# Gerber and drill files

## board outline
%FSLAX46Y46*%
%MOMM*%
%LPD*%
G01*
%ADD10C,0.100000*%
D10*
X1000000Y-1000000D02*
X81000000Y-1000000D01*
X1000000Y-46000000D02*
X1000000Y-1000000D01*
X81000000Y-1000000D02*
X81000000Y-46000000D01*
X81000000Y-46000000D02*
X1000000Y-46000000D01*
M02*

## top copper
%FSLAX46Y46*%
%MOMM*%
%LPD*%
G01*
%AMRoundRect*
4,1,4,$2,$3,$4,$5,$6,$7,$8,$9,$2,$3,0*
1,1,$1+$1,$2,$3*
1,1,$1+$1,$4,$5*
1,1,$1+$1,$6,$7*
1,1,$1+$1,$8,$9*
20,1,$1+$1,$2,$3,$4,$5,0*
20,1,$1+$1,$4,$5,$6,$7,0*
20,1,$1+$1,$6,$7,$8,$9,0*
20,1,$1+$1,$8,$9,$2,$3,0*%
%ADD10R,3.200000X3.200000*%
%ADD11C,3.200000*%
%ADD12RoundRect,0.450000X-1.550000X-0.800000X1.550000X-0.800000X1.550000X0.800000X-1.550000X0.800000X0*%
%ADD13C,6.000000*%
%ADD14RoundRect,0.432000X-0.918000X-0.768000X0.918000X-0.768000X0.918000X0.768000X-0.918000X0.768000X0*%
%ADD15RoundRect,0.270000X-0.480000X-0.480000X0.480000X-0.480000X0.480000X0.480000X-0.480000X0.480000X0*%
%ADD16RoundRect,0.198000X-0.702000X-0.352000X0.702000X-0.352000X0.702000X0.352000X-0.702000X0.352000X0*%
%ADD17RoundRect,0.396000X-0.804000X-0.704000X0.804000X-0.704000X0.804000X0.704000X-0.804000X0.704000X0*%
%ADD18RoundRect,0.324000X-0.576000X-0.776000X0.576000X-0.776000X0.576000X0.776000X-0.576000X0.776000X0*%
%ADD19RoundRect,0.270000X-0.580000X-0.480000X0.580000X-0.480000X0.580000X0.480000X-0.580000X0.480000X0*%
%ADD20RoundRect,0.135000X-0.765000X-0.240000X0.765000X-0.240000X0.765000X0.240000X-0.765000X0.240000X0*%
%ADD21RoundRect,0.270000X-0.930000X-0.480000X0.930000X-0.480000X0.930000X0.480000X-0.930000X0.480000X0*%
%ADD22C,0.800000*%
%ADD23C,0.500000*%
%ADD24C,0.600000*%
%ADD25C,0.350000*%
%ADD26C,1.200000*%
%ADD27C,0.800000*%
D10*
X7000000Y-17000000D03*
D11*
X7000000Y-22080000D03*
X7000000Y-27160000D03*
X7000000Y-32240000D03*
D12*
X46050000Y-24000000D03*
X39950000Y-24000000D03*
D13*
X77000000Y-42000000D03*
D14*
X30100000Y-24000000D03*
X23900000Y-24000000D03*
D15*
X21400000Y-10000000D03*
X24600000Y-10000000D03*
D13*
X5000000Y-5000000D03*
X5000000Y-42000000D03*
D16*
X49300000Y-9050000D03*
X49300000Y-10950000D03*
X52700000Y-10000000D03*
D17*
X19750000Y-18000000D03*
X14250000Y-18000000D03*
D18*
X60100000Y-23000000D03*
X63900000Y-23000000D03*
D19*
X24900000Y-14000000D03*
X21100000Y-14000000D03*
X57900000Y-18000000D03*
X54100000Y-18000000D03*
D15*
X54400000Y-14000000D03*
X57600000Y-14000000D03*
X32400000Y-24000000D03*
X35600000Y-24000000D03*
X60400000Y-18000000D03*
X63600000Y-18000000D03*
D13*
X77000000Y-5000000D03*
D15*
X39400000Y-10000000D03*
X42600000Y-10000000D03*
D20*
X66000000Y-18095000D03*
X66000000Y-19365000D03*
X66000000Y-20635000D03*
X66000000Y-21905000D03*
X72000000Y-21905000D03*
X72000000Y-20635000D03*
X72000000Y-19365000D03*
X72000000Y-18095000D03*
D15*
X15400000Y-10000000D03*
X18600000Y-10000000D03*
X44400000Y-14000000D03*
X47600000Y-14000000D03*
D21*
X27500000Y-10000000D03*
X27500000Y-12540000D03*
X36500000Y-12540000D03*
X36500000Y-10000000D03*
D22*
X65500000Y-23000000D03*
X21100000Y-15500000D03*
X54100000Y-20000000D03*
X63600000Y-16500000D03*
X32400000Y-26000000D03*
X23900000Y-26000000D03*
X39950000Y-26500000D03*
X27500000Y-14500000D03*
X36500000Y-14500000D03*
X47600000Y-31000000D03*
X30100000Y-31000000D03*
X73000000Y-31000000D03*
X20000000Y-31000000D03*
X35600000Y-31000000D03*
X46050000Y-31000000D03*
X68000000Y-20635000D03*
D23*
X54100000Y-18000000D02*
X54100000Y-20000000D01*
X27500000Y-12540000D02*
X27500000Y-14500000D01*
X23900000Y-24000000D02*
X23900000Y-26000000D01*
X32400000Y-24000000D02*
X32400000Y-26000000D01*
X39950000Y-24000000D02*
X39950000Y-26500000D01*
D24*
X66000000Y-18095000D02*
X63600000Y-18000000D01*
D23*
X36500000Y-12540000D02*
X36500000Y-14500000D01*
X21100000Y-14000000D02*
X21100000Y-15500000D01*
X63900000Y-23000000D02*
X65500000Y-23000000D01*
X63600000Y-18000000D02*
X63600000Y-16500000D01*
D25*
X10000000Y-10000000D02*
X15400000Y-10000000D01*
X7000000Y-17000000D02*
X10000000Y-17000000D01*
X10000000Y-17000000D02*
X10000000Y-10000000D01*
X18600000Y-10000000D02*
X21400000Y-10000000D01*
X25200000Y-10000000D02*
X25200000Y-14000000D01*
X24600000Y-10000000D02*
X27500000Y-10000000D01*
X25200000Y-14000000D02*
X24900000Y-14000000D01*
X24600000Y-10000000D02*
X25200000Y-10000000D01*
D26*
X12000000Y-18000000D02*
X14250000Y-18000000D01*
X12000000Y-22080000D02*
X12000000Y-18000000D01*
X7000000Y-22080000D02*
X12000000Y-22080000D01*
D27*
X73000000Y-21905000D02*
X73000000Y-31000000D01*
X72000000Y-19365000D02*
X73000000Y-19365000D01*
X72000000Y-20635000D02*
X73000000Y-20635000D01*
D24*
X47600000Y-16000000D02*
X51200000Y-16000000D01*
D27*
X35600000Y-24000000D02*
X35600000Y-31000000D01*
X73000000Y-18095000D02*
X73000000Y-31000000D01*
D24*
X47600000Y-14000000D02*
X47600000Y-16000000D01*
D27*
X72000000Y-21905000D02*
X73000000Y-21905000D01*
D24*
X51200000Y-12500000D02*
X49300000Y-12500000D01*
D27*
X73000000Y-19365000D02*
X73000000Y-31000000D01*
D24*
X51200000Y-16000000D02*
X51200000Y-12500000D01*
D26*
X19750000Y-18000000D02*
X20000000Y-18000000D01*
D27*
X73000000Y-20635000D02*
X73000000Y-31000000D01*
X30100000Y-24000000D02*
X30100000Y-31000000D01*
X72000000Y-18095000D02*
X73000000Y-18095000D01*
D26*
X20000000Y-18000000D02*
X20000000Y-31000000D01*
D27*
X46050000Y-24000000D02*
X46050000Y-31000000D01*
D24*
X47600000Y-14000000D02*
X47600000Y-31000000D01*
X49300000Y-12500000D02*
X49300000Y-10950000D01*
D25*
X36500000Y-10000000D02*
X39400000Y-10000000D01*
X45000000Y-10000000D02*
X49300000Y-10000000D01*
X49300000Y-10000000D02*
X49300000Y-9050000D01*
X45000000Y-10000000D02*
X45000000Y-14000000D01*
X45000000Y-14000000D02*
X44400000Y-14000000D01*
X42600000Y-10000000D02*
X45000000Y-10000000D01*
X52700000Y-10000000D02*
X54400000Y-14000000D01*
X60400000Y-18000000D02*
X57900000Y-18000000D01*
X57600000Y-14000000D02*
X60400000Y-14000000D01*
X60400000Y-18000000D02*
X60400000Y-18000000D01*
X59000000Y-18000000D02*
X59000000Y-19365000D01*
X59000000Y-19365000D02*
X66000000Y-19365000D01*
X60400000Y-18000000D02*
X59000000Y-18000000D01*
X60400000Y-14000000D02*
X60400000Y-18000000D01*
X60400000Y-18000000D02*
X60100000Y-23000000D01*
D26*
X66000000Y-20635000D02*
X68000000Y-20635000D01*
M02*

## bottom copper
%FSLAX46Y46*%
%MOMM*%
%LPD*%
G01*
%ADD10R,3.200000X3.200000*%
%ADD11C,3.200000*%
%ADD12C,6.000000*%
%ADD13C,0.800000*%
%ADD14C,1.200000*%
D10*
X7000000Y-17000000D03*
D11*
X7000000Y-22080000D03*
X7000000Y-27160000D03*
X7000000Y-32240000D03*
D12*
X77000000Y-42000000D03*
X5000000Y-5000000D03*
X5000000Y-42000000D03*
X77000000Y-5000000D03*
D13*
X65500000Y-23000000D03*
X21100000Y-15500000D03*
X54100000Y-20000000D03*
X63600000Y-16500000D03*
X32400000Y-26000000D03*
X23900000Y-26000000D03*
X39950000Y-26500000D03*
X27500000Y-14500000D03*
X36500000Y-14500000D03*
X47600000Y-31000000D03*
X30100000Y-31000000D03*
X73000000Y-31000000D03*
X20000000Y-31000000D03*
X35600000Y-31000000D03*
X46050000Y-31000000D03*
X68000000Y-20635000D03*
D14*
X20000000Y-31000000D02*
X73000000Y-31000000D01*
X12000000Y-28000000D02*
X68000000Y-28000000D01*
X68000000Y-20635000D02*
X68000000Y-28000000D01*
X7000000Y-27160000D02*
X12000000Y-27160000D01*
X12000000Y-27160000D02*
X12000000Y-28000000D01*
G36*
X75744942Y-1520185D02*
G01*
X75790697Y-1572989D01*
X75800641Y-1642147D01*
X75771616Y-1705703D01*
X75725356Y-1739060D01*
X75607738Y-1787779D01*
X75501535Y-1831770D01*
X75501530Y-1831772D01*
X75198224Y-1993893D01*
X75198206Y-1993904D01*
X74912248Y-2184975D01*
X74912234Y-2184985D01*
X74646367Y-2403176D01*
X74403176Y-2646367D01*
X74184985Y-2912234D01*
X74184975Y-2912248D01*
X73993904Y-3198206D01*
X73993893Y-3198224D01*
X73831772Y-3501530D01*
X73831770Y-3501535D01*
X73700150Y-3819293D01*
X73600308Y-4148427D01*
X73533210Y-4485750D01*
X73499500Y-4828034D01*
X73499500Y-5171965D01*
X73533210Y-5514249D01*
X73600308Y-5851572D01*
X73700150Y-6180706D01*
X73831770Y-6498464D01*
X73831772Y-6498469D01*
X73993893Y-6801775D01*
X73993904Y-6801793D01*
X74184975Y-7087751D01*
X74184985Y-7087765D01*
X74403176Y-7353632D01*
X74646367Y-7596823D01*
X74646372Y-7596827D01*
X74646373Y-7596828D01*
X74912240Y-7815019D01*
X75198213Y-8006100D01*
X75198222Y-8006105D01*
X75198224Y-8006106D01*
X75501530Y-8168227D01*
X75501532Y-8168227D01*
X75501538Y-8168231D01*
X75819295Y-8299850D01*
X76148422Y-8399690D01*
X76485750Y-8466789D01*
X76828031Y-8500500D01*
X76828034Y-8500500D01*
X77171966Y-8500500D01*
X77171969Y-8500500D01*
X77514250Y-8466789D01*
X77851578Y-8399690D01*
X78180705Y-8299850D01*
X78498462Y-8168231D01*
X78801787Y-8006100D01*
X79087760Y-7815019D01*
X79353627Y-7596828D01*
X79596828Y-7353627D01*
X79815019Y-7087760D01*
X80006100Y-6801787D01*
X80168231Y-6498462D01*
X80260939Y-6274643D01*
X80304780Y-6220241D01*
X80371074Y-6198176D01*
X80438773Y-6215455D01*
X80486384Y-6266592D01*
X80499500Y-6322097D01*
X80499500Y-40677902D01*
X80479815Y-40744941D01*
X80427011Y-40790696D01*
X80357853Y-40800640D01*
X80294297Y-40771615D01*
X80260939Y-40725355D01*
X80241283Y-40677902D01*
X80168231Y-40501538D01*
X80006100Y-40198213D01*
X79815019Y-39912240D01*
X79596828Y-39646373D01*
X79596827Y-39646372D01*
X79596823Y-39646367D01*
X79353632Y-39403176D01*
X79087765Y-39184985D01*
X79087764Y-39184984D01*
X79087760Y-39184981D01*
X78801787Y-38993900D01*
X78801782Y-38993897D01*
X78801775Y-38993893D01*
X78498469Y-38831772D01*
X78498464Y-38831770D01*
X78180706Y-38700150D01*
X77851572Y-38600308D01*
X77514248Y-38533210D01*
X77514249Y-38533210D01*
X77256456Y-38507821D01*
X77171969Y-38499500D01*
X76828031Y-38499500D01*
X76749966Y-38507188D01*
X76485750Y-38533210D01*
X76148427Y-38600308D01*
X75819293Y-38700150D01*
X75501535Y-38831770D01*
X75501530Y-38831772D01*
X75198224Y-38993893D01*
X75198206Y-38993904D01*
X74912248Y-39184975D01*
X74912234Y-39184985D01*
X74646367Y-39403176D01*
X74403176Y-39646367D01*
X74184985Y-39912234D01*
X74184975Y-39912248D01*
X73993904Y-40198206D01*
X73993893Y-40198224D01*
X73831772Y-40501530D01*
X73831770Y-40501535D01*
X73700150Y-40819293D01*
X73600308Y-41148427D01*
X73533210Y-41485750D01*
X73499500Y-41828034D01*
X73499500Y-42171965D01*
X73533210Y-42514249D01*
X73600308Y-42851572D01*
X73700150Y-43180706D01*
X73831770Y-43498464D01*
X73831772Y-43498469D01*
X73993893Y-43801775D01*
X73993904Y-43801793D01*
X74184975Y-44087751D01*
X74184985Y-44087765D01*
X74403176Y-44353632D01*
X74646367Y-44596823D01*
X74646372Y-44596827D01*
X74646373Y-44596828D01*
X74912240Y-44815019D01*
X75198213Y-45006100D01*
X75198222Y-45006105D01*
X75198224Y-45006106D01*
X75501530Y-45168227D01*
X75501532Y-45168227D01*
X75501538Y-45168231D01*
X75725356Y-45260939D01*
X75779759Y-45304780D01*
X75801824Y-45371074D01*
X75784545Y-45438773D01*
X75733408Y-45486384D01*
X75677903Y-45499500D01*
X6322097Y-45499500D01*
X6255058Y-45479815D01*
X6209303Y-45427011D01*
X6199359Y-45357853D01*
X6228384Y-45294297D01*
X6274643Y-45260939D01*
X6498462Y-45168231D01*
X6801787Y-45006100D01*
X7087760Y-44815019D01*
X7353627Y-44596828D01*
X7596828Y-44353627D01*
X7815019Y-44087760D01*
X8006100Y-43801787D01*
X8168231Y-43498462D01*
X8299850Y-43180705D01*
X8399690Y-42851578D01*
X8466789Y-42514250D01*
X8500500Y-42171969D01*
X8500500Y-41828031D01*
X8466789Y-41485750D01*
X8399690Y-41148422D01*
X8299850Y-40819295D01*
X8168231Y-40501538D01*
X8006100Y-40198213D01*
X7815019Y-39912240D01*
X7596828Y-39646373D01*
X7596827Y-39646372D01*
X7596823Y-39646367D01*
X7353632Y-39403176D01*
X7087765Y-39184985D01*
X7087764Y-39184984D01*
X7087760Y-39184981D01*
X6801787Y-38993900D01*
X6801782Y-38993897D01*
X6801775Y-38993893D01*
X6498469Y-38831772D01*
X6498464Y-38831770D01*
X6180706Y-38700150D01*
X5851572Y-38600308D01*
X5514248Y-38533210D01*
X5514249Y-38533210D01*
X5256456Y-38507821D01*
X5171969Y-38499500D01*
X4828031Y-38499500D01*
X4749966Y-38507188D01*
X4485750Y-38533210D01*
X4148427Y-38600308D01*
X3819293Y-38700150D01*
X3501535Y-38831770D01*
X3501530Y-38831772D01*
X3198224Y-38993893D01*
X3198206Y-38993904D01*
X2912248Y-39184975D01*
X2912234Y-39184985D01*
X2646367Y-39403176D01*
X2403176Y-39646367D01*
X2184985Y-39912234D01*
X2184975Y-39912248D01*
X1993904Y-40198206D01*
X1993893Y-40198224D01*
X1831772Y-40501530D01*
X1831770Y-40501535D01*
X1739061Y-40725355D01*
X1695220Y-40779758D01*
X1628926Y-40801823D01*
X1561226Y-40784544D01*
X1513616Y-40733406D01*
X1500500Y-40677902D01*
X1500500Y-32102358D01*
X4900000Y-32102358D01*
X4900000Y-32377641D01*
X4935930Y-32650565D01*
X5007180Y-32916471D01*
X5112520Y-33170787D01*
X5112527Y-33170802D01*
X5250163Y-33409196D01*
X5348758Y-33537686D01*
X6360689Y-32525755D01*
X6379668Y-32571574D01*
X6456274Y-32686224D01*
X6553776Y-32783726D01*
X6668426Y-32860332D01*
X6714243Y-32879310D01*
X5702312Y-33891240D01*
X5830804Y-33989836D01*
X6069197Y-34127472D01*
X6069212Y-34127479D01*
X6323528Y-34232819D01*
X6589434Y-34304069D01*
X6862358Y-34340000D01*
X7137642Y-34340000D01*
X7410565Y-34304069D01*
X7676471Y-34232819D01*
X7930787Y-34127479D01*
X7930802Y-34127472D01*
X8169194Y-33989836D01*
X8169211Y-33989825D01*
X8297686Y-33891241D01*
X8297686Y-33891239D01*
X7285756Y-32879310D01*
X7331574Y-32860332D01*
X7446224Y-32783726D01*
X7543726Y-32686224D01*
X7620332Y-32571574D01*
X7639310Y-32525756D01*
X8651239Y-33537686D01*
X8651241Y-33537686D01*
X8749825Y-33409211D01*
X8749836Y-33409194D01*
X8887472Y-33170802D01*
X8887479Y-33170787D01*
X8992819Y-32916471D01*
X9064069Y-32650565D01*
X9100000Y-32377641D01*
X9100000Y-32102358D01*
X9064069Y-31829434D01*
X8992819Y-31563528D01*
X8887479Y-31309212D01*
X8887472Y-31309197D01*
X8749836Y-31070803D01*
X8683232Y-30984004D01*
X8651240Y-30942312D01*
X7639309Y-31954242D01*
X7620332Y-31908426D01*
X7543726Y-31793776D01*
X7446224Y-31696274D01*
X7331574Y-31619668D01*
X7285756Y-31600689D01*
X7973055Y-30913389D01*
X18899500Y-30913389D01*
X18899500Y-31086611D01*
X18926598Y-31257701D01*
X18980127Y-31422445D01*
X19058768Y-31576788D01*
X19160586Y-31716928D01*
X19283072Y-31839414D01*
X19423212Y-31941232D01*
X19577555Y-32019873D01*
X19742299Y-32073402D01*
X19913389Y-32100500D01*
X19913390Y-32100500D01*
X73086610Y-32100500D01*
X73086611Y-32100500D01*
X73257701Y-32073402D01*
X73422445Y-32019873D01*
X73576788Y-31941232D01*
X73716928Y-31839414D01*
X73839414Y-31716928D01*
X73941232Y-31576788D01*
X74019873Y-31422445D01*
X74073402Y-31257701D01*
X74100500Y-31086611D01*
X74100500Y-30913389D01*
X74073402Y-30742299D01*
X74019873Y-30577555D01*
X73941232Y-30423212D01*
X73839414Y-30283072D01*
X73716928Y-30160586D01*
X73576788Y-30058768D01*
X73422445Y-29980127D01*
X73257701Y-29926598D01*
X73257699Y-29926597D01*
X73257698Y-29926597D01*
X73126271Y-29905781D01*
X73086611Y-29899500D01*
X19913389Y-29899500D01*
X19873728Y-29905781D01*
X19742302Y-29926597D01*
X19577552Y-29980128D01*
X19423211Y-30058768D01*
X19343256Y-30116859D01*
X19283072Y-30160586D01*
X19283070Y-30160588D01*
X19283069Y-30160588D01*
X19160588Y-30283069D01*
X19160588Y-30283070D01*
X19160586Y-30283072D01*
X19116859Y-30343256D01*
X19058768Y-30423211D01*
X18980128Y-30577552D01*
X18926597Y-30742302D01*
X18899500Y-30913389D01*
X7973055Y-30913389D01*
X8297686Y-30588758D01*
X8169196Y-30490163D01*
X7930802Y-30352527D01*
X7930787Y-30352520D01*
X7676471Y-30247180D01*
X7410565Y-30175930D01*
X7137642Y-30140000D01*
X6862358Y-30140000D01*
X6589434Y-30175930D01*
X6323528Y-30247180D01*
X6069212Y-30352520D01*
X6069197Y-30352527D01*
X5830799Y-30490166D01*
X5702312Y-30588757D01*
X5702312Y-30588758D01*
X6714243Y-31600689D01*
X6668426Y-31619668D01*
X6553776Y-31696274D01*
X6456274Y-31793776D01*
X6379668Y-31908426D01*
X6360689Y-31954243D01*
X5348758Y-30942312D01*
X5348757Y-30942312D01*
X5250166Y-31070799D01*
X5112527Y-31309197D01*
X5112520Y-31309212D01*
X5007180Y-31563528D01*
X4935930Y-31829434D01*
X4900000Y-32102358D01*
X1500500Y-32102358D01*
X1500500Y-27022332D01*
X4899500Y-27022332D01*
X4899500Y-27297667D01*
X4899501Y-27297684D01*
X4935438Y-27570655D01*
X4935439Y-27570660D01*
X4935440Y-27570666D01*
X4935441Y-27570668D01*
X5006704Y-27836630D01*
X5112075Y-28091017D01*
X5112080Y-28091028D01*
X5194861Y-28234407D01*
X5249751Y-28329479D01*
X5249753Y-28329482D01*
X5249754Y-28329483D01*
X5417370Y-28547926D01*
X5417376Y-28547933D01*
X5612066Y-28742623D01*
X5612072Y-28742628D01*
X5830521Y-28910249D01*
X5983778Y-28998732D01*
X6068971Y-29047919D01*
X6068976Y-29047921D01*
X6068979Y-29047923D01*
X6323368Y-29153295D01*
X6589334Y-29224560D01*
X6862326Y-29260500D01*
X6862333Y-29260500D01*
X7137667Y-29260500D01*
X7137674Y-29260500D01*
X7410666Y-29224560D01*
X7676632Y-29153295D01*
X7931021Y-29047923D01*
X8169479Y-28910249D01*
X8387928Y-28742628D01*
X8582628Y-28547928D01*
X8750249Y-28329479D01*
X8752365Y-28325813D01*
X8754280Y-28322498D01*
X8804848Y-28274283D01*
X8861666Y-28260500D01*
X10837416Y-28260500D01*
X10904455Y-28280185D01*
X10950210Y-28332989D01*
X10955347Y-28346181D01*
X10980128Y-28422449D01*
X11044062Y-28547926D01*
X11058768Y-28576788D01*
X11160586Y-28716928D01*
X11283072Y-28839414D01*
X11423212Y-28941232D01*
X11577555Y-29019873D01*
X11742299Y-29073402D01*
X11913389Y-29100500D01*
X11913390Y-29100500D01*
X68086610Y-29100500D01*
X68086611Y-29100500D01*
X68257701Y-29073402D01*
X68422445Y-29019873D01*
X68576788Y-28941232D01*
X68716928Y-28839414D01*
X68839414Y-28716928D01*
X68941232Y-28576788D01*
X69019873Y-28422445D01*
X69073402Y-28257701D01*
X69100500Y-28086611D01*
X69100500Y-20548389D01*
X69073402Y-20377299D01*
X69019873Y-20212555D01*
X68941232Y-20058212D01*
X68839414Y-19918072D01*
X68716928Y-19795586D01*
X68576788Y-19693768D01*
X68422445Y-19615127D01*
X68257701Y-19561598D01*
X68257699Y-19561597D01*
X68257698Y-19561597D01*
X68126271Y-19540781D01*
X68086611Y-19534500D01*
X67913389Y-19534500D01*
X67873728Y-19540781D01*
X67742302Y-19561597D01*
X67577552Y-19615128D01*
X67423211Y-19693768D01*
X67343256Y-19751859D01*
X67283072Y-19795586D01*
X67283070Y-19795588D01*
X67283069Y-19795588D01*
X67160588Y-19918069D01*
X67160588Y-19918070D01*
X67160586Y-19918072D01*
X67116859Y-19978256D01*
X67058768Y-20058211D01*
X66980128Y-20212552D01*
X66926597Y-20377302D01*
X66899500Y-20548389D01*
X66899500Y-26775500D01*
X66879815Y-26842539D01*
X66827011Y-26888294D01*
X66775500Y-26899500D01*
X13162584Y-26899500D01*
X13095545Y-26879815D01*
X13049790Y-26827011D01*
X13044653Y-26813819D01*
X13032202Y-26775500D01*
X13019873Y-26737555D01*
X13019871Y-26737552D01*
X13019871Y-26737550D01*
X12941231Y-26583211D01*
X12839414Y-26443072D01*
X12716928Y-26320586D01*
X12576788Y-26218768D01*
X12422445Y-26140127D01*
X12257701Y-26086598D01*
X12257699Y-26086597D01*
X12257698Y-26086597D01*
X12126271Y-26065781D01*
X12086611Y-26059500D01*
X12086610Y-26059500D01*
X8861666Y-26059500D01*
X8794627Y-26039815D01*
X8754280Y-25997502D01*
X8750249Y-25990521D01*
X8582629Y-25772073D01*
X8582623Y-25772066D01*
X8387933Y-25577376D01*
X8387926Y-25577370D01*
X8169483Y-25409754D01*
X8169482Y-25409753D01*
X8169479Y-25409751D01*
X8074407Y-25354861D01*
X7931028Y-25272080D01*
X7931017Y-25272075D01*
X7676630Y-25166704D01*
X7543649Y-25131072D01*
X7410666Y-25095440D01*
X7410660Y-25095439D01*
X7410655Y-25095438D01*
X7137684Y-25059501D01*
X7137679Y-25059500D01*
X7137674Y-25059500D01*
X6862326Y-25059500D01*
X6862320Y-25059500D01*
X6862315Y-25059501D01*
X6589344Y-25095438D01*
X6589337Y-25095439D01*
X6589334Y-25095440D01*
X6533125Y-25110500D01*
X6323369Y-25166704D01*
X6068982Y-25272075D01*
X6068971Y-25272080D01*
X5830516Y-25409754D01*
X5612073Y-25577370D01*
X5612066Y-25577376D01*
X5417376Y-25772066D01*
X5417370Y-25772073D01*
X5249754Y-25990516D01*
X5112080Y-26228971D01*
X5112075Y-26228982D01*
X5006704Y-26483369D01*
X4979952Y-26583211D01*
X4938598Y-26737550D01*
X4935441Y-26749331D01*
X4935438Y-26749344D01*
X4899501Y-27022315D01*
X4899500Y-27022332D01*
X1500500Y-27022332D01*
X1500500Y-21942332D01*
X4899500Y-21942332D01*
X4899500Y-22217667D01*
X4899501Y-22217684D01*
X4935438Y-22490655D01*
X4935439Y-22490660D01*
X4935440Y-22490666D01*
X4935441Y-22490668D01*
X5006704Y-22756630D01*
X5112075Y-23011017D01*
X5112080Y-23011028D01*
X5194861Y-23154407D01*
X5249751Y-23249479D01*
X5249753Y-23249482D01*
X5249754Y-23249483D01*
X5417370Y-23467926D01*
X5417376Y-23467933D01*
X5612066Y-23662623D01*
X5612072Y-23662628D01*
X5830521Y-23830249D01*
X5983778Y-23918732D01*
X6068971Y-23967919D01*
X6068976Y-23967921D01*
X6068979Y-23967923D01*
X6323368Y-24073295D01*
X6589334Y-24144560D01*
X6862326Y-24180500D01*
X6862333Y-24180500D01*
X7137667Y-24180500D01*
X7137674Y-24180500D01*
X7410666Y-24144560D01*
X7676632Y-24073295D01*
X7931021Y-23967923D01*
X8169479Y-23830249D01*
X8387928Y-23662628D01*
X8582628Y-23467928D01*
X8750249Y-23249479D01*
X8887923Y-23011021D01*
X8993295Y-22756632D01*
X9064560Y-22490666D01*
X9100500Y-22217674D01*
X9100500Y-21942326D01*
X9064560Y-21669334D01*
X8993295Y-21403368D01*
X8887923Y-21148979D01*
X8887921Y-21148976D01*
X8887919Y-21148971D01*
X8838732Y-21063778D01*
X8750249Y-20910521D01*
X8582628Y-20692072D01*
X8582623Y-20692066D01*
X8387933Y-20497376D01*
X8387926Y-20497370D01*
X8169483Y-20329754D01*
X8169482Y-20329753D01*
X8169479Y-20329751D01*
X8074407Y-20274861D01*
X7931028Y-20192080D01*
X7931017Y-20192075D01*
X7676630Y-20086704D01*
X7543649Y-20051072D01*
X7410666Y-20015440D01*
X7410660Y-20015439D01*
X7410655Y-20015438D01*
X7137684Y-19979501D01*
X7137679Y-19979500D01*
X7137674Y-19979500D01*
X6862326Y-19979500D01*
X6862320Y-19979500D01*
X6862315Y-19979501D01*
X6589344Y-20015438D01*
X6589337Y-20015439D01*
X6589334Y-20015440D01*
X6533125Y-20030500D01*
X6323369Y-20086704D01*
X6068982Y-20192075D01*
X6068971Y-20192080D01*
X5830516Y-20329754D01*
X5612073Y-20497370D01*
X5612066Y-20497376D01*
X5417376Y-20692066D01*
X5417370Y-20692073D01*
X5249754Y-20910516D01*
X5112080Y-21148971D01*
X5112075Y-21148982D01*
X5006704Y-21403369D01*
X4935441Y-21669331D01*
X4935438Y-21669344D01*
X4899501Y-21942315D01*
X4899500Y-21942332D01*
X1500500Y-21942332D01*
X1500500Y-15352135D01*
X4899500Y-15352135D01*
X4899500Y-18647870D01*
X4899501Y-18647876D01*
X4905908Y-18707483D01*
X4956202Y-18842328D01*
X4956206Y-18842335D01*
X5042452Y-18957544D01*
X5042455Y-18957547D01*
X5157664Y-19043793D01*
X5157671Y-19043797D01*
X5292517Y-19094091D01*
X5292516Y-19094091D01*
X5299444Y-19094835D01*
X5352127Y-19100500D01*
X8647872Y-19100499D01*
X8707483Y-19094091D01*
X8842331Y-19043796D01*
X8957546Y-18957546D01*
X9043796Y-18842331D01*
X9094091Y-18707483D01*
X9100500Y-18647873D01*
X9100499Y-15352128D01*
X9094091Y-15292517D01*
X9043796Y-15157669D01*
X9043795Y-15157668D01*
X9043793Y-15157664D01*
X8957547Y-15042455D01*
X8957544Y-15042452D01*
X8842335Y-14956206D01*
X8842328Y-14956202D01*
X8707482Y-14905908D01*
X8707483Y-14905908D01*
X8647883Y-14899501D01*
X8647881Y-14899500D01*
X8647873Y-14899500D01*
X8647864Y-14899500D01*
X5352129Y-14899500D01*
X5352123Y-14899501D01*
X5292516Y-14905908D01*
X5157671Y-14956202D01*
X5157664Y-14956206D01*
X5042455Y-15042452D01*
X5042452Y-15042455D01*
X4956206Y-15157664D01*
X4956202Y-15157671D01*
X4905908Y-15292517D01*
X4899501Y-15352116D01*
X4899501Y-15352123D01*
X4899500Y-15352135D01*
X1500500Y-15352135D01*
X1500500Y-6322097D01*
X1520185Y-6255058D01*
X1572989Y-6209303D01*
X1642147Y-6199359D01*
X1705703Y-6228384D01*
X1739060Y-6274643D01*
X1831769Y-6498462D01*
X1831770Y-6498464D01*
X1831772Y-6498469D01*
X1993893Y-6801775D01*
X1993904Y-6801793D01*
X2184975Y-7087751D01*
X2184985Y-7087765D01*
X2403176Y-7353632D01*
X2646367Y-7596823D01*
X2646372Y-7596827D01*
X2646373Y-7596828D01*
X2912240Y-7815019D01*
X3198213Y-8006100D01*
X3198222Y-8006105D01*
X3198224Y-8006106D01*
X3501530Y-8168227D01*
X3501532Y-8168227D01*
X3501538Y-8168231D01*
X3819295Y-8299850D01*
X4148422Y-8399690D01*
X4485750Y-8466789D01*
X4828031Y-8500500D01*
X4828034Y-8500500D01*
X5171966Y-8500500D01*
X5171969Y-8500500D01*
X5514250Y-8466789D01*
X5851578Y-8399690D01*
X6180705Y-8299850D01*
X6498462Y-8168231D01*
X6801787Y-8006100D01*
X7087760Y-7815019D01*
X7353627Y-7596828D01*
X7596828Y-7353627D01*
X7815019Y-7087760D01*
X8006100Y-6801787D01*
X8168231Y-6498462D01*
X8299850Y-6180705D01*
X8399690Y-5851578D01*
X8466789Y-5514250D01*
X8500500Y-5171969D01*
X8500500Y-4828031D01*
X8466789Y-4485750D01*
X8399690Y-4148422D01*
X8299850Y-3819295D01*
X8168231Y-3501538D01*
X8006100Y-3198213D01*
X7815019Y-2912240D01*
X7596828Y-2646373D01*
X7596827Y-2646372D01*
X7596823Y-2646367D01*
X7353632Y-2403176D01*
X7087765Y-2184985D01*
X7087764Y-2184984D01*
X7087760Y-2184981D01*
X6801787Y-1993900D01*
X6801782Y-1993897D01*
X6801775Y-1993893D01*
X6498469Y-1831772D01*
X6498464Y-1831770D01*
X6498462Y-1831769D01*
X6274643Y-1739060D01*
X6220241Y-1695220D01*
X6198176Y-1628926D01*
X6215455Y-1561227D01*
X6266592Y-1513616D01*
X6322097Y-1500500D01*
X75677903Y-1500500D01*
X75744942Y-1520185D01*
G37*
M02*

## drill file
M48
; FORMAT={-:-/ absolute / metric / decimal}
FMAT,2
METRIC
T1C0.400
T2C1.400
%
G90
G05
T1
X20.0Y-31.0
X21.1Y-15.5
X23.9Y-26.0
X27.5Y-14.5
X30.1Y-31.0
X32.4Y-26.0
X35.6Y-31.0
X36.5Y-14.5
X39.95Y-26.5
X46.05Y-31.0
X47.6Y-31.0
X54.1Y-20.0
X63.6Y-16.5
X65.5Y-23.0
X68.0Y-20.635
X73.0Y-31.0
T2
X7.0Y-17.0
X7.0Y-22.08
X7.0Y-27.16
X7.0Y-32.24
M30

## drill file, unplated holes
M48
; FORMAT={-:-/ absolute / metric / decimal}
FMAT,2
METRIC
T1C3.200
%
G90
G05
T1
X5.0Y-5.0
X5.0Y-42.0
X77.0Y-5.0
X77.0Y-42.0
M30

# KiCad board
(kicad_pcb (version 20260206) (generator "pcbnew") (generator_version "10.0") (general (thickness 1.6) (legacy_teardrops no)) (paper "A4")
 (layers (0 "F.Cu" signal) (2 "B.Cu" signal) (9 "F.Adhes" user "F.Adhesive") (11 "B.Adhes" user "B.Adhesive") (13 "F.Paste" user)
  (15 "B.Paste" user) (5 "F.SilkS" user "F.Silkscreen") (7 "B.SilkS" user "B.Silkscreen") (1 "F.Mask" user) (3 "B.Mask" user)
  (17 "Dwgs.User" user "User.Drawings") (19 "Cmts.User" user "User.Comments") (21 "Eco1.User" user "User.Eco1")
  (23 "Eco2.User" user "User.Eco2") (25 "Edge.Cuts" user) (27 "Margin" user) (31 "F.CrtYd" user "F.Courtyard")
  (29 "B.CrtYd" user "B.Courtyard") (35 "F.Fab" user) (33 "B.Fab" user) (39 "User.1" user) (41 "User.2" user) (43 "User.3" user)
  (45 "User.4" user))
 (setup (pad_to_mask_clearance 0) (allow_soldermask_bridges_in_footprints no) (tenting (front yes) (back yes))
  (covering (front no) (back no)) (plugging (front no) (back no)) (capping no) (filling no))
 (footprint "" (layer "F.Cu") (at 0 0)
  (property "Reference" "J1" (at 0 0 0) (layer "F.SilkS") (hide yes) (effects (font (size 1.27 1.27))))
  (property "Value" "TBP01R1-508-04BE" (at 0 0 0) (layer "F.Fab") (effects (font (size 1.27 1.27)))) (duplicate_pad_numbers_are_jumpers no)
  (pad "1" thru_hole rect (at 7 17) (size 3.2 3.2) (drill 1.4) (layers "*.Cu" "*.Mask") (remove_unused_layers no) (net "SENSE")
   (thermal_bridge_angle 45))
  (pad "2" thru_hole circle (at 7 22.08) (size 3.2 3.2) (drill 1.4) (layers "*.Cu" "*.Mask") (remove_unused_layers no) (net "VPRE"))
  (pad "3" thru_hole circle (at 7 27.16) (size 3.2 3.2) (drill 1.4) (layers "*.Cu" "*.Mask") (remove_unused_layers no) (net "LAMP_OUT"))
  (pad "4" thru_hole circle (at 7 32.24) (size 3.2 3.2) (drill 1.4) (layers "*.Cu" "*.Mask") (remove_unused_layers no) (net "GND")))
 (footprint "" (layer "F.Cu") (at 0 0)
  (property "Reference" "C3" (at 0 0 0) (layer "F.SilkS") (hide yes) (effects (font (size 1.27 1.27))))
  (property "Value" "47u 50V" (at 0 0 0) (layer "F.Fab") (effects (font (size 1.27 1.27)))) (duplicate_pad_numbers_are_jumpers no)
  (pad "1" smd roundrect (at 46.05 24) (size 4 2.5) (layers "F.Cu" "F.Mask" "F.Paste") (roundrect_rratio 0.18) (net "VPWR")
   (thermal_bridge_angle 45))
  (pad "2" smd roundrect (at 39.95 24) (size 4 2.5) (layers "F.Cu" "F.Mask" "F.Paste") (roundrect_rratio 0.18) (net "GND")
   (thermal_bridge_angle 45)))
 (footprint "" (layer "F.Cu") (at 0 0)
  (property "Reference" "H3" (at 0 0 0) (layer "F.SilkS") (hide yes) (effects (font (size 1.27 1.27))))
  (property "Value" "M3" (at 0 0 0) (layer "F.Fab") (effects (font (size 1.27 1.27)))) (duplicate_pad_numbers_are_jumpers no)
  (pad "" np_thru_hole circle (at 77 42) (size 6 6) (drill 3.2) (layers "*.Cu" "*.Mask")))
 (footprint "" (layer "F.Cu") (at 0 0)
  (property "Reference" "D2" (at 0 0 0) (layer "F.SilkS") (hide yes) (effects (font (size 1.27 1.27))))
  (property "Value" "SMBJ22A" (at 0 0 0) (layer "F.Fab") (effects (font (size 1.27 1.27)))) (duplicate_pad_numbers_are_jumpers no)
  (pad "1" smd roundrect (at 30.1 24) (size 2.7 2.4) (layers "F.Cu" "F.Mask" "F.Paste") (roundrect_rratio 0.18) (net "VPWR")
   (thermal_bridge_angle 45))
  (pad "2" smd roundrect (at 23.9 24) (size 2.7 2.4) (layers "F.Cu" "F.Mask" "F.Paste") (roundrect_rratio 0.18) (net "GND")
   (thermal_bridge_angle 45)))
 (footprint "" (layer "F.Cu") (at 0 0)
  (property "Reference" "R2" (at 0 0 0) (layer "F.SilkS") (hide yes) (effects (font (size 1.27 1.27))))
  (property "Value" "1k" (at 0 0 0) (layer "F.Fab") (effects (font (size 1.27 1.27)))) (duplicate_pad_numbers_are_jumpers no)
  (pad "1" smd roundrect (at 21.4 10) (size 1.5 1.5) (layers "F.Cu" "F.Mask" "F.Paste") (roundrect_rratio 0.18) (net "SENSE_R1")
   (thermal_bridge_angle 45))
  (pad "2" smd roundrect (at 24.6 10) (size 1.5 1.5) (layers "F.Cu" "F.Mask" "F.Paste") (roundrect_rratio 0.18) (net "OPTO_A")
   (thermal_bridge_angle 45)))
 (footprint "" (layer "F.Cu") (at 0 0)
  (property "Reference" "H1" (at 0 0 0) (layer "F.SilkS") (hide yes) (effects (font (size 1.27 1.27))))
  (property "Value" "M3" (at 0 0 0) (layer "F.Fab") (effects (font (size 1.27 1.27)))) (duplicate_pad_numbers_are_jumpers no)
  (pad "" np_thru_hole circle (at 5 5) (size 6 6) (drill 3.2) (layers "*.Cu" "*.Mask")))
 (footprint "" (layer "F.Cu") (at 0 0)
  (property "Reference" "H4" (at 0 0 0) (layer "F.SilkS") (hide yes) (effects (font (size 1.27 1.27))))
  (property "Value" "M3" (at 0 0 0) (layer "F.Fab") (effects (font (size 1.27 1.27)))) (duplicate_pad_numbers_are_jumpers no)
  (pad "" np_thru_hole circle (at 5 42) (size 6 6) (drill 3.2) (layers "*.Cu" "*.Mask")))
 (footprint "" (layer "F.Cu") (at 0 0)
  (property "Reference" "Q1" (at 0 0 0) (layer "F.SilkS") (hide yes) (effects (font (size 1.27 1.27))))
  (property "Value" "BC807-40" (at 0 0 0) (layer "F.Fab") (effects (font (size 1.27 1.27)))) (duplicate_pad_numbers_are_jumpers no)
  (pad "1" smd roundrect (at 49.3 9.05) (size 1.8 1.1) (layers "F.Cu" "F.Mask" "F.Paste") (roundrect_rratio 0.18) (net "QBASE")
   (thermal_bridge_angle 45))
  (pad "2" smd roundrect (at 49.3 10.95) (size 1.8 1.1) (layers "F.Cu" "F.Mask" "F.Paste") (roundrect_rratio 0.18) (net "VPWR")
   (thermal_bridge_angle 45))
  (pad "3" smd roundrect (at 52.7 10) (size 1.8 1.1) (layers "F.Cu" "F.Mask" "F.Paste") (roundrect_rratio 0.18) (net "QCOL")
   (thermal_bridge_angle 45)))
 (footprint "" (layer "F.Cu") (at 0 0)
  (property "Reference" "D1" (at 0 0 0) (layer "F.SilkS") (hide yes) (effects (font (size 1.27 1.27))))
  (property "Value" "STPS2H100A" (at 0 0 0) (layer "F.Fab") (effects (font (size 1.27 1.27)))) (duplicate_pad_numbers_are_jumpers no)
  (pad "1" smd roundrect (at 19.75 18) (size 2.4 2.2) (layers "F.Cu" "F.Mask" "F.Paste") (roundrect_rratio 0.18) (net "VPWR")
   (thermal_bridge_angle 45))
  (pad "2" smd roundrect (at 14.25 18) (size 2.4 2.2) (layers "F.Cu" "F.Mask" "F.Paste") (roundrect_rratio 0.18) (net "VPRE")
   (thermal_bridge_angle 45)))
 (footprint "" (layer "F.Cu") (at 0 0)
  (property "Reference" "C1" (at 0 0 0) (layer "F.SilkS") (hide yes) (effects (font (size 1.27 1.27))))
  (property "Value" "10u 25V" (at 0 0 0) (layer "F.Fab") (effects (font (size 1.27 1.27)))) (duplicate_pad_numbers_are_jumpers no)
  (pad "1" smd roundrect (at 60.1 23) (size 1.8 2.2) (layers "F.Cu" "F.Mask" "F.Paste") (roundrect_rratio 0.18) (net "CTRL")
   (thermal_bridge_angle 45))
  (pad "2" smd roundrect (at 63.9 23) (size 1.8 2.2) (layers "F.Cu" "F.Mask" "F.Paste") (roundrect_rratio 0.18) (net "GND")
   (thermal_bridge_angle 45)))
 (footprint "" (layer "F.Cu") (at 0 0)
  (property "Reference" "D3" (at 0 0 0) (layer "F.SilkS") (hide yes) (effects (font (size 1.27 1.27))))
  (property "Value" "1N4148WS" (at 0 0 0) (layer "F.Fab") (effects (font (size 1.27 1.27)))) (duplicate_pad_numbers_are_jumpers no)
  (pad "1" smd roundrect (at 24.9 14) (size 1.7 1.5) (layers "F.Cu" "F.Mask" "F.Paste") (roundrect_rratio 0.18) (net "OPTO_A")
   (thermal_bridge_angle 45))
  (pad "2" smd roundrect (at 21.1 14) (size 1.7 1.5) (layers "F.Cu" "F.Mask" "F.Paste") (roundrect_rratio 0.18) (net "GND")
   (thermal_bridge_angle 45)))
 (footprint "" (layer "F.Cu") (at 0 0)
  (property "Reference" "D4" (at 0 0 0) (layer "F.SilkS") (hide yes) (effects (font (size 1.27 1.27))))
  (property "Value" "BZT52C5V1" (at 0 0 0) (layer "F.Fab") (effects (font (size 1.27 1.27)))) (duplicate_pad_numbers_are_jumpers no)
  (pad "1" smd roundrect (at 57.9 18) (size 1.7 1.5) (layers "F.Cu" "F.Mask" "F.Paste") (roundrect_rratio 0.18) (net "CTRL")
   (thermal_bridge_angle 45))
  (pad "2" smd roundrect (at 54.1 18) (size 1.7 1.5) (layers "F.Cu" "F.Mask" "F.Paste") (roundrect_rratio 0.18) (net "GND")
   (thermal_bridge_angle 45)))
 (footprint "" (layer "F.Cu") (at 0 0)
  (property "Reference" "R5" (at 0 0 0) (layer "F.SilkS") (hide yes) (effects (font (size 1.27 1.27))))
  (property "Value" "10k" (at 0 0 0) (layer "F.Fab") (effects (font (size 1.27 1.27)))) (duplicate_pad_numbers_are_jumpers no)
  (pad "1" smd roundrect (at 54.4 14) (size 1.5 1.5) (layers "F.Cu" "F.Mask" "F.Paste") (roundrect_rratio 0.18) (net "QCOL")
   (thermal_bridge_angle 45))
  (pad "2" smd roundrect (at 57.6 14) (size 1.5 1.5) (layers "F.Cu" "F.Mask" "F.Paste") (roundrect_rratio 0.18) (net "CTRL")
   (thermal_bridge_angle 45)))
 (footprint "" (layer "F.Cu") (at 0 0)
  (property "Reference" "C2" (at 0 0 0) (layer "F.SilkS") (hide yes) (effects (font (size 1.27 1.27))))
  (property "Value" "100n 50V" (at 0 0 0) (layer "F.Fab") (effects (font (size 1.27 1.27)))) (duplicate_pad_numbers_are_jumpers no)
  (pad "1" smd roundrect (at 32.4 24) (size 1.5 1.5) (layers "F.Cu" "F.Mask" "F.Paste") (roundrect_rratio 0.18) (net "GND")
   (thermal_bridge_angle 45))
  (pad "2" smd roundrect (at 35.6 24) (size 1.5 1.5) (layers "F.Cu" "F.Mask" "F.Paste") (roundrect_rratio 0.18) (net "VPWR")
   (thermal_bridge_angle 45)))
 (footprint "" (layer "F.Cu") (at 0 0)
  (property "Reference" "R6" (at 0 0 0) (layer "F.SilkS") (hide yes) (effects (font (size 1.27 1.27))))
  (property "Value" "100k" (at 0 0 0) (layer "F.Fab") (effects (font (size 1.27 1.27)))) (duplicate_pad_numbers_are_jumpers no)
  (pad "1" smd roundrect (at 60.4 18) (size 1.5 1.5) (layers "F.Cu" "F.Mask" "F.Paste") (roundrect_rratio 0.18) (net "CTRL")
   (thermal_bridge_angle 45))
  (pad "2" smd roundrect (at 63.6 18) (size 1.5 1.5) (layers "F.Cu" "F.Mask" "F.Paste") (roundrect_rratio 0.18) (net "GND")
   (thermal_bridge_angle 45)))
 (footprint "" (layer "F.Cu") (at 0 0)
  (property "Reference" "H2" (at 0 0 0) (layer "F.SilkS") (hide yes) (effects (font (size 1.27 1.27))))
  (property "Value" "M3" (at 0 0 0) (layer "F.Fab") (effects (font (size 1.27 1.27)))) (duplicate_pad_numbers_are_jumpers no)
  (pad "" np_thru_hole circle (at 77 5) (size 6 6) (drill 3.2) (layers "*.Cu" "*.Mask")))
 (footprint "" (layer "F.Cu") (at 0 0)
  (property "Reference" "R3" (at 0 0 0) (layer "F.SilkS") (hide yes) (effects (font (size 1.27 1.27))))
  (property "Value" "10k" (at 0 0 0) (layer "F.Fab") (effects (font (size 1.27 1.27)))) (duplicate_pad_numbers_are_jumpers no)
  (pad "1" smd roundrect (at 39.4 10) (size 1.5 1.5) (layers "F.Cu" "F.Mask" "F.Paste") (roundrect_rratio 0.18) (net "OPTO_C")
   (thermal_bridge_angle 45))
  (pad "2" smd roundrect (at 42.6 10) (size 1.5 1.5) (layers "F.Cu" "F.Mask" "F.Paste") (roundrect_rratio 0.18) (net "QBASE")
   (thermal_bridge_angle 45)))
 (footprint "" (layer "F.Cu") (at 0 0)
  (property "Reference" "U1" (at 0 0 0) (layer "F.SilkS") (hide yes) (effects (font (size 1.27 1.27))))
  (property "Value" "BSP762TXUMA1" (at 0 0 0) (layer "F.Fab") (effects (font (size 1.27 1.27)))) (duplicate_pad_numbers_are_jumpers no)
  (pad "1" smd roundrect (at 66 18.095) (size 1.8 0.75) (layers "F.Cu" "F.Mask" "F.Paste") (roundrect_rratio 0.18) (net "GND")
   (thermal_bridge_angle 45))
  (pad "2" smd roundrect (at 66 19.365) (size 1.8 0.75) (layers "F.Cu" "F.Mask" "F.Paste") (roundrect_rratio 0.18) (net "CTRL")
   (thermal_bridge_angle 45))
  (pad "3" smd roundrect (at 66 20.635) (size 1.8 0.75) (layers "F.Cu" "F.Mask" "F.Paste") (roundrect_rratio 0.18) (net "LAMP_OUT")
   (thermal_bridge_angle 45))
  (pad "4" smd roundrect (at 66 21.905) (size 1.8 0.75) (layers "F.Cu" "F.Mask" "F.Paste") (roundrect_rratio 0.18) (thermal_bridge_angle 45))
  (pad "5" smd roundrect (at 72 21.905) (size 1.8 0.75) (layers "F.Cu" "F.Mask" "F.Paste") (roundrect_rratio 0.18) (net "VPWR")
   (thermal_bridge_angle 45))
  (pad "6" smd roundrect (at 72 20.635) (size 1.8 0.75) (layers "F.Cu" "F.Mask" "F.Paste") (roundrect_rratio 0.18) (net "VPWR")
   (thermal_bridge_angle 45))
  (pad "7" smd roundrect (at 72 19.365) (size 1.8 0.75) (layers "F.Cu" "F.Mask" "F.Paste") (roundrect_rratio 0.18) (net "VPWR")
   (thermal_bridge_angle 45))
  (pad "8" smd roundrect (at 72 18.095) (size 1.8 0.75) (layers "F.Cu" "F.Mask" "F.Paste") (roundrect_rratio 0.18) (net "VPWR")
   (thermal_bridge_angle 45)))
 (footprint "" (layer "F.Cu") (at 0 0)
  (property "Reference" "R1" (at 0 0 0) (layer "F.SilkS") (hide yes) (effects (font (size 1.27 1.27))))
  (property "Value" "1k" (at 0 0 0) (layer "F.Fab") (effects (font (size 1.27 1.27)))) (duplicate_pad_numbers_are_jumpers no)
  (pad "1" smd roundrect (at 15.4 10) (size 1.5 1.5) (layers "F.Cu" "F.Mask" "F.Paste") (roundrect_rratio 0.18) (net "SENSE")
   (thermal_bridge_angle 45))
  (pad "2" smd roundrect (at 18.6 10) (size 1.5 1.5) (layers "F.Cu" "F.Mask" "F.Paste") (roundrect_rratio 0.18) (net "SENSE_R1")
   (thermal_bridge_angle 45)))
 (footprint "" (layer "F.Cu") (at 0 0)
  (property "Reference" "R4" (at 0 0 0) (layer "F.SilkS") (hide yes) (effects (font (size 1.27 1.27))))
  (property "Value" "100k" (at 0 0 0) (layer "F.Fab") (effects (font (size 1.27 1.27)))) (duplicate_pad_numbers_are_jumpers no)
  (pad "1" smd roundrect (at 44.4 14) (size 1.5 1.5) (layers "F.Cu" "F.Mask" "F.Paste") (roundrect_rratio 0.18) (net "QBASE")
   (thermal_bridge_angle 45))
  (pad "2" smd roundrect (at 47.6 14) (size 1.5 1.5) (layers "F.Cu" "F.Mask" "F.Paste") (roundrect_rratio 0.18) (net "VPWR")
   (thermal_bridge_angle 45)))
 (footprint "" (layer "F.Cu") (at 0 0)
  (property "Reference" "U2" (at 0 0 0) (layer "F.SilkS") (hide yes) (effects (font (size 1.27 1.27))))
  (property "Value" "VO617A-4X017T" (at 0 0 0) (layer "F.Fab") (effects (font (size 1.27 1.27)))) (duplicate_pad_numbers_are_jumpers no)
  (pad "1" smd roundrect (at 27.5 10) (size 2.4 1.5) (layers "F.Cu" "F.Mask" "F.Paste") (roundrect_rratio 0.18) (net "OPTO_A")
   (thermal_bridge_angle 45))
  (pad "2" smd roundrect (at 27.5 12.54) (size 2.4 1.5) (layers "F.Cu" "F.Mask" "F.Paste") (roundrect_rratio 0.18) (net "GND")
   (thermal_bridge_angle 45))
  (pad "3" smd roundrect (at 36.5 12.54) (size 2.4 1.5) (layers "F.Cu" "F.Mask" "F.Paste") (roundrect_rratio 0.18) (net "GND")
   (thermal_bridge_angle 45))
  (pad "4" smd roundrect (at 36.5 10) (size 2.4 1.5) (layers "F.Cu" "F.Mask" "F.Paste") (roundrect_rratio 0.18) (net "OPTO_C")
   (thermal_bridge_angle 45)))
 (gr_line (start 1 1) (end 81 1) (stroke (width 0.1) (type default)) (layer "Edge.Cuts"))
 (gr_line (start 1 46) (end 1 1) (stroke (width 0.1) (type default)) (layer "Edge.Cuts"))
 (gr_line (start 81 1) (end 81 46) (stroke (width 0.1) (type default)) (layer "Edge.Cuts"))
 (gr_line (start 81 46) (end 1 46) (stroke (width 0.1) (type default)) (layer "Edge.Cuts"))
 (segment (start 54.1 18) (end 54.1 20) (width 0.5) (layer "F.Cu") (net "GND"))
 (segment (start 27.5 12.54) (end 27.5 14.5) (width 0.5) (layer "F.Cu") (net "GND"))
 (segment (start 23.9 24) (end 23.9 26) (width 0.5) (layer "F.Cu") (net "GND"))
 (segment (start 32.4 24) (end 32.4 26) (width 0.5) (layer "F.Cu") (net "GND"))
 (segment (start 39.95 24) (end 39.95 26.5) (width 0.5) (layer "F.Cu") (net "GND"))
 (segment (start 66 18.095) (end 63.6 18) (width 0.6) (layer "F.Cu") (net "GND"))
 (segment (start 36.5 12.54) (end 36.5 14.5) (width 0.5) (layer "F.Cu") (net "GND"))
 (segment (start 21.1 14) (end 21.1 15.5) (width 0.5) (layer "F.Cu") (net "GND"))
 (segment (start 63.9 23) (end 65.5 23) (width 0.5) (layer "F.Cu") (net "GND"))
 (segment (start 63.6 18) (end 63.6 16.5) (width 0.5) (layer "F.Cu") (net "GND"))
 (via (at 65.5 23) (size 0.8) (drill 0.4) (layers "F.Cu" "B.Cu") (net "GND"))
 (via (at 21.1 15.5) (size 0.8) (drill 0.4) (layers "F.Cu" "B.Cu") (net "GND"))
 (via (at 54.1 20) (size 0.8) (drill 0.4) (layers "F.Cu" "B.Cu") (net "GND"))
 (via (at 63.6 16.5) (size 0.8) (drill 0.4) (layers "F.Cu" "B.Cu") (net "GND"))
 (via (at 32.4 26) (size 0.8) (drill 0.4) (layers "F.Cu" "B.Cu") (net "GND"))
 (via (at 23.9 26) (size 0.8) (drill 0.4) (layers "F.Cu" "B.Cu") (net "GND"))
 (via (at 39.95 26.5) (size 0.8) (drill 0.4) (layers "F.Cu" "B.Cu") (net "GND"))
 (via (at 27.5 14.5) (size 0.8) (drill 0.4) (layers "F.Cu" "B.Cu") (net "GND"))
 (via (at 36.5 14.5) (size 0.8) (drill 0.4) (layers "F.Cu" "B.Cu") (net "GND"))
 (segment (start 10 10) (end 15.4 10) (width 0.35) (layer "F.Cu") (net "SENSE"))
 (segment (start 7 17) (end 10 17) (width 0.35) (layer "F.Cu") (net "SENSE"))
 (segment (start 10 17) (end 10 10) (width 0.35) (layer "F.Cu") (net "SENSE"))
 (segment (start 18.6 10) (end 21.4 10) (width 0.35) (layer "F.Cu") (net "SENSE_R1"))
 (segment (start 25.2 10) (end 25.2 14) (width 0.35) (layer "F.Cu") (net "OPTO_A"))
 (segment (start 24.6 10) (end 27.5 10) (width 0.35) (layer "F.Cu") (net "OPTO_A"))
 (segment (start 25.2 14) (end 24.9 14) (width 0.35) (layer "F.Cu") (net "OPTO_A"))
 (segment (start 24.6 10) (end 25.2 10) (width 0.35) (layer "F.Cu") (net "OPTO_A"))
 (segment (start 12 18) (end 14.25 18) (width 1.2) (layer "F.Cu") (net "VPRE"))
 (segment (start 12 22.08) (end 12 18) (width 1.2) (layer "F.Cu") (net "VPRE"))
 (segment (start 7 22.08) (end 12 22.08) (width 1.2) (layer "F.Cu") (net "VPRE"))
 (segment (start 73 21.905) (end 73 31) (width 0.8) (layer "F.Cu") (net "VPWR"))
 (segment (start 72 19.365) (end 73 19.365) (width 0.8) (layer "F.Cu") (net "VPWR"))
 (segment (start 72 20.635) (end 73 20.635) (width 0.8) (layer "F.Cu") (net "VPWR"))
 (segment (start 47.6 16) (end 51.2 16) (width 0.6) (layer "F.Cu") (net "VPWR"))
 (segment (start 35.6 24) (end 35.6 31) (width 0.8) (layer "F.Cu") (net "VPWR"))
 (segment (start 73 18.095) (end 73 31) (width 0.8) (layer "F.Cu") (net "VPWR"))
 (segment (start 47.6 14) (end 47.6 16) (width 0.6) (layer "F.Cu") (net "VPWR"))
 (segment (start 72 21.905) (end 73 21.905) (width 0.8) (layer "F.Cu") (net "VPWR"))
 (segment (start 51.2 12.5) (end 49.3 12.5) (width 0.6) (layer "F.Cu") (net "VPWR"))
 (segment (start 73 19.365) (end 73 31) (width 0.8) (layer "F.Cu") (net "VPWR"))
 (segment (start 51.2 16) (end 51.2 12.5) (width 0.6) (layer "F.Cu") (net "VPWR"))
 (segment (start 19.75 18) (end 20 18) (width 1.2) (layer "F.Cu") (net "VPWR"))
 (segment (start 73 20.635) (end 73 31) (width 0.8) (layer "F.Cu") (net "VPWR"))
 (segment (start 30.1 24) (end 30.1 31) (width 0.8) (layer "F.Cu") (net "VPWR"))
 (segment (start 72 18.095) (end 73 18.095) (width 0.8) (layer "F.Cu") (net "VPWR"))
 (segment (start 20 18) (end 20 31) (width 1.2) (layer "F.Cu") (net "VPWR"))
 (segment (start 46.05 24) (end 46.05 31) (width 0.8) (layer "F.Cu") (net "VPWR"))
 (segment (start 47.6 14) (end 47.6 31) (width 0.6) (layer "F.Cu") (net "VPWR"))
 (segment (start 49.3 12.5) (end 49.3 10.95) (width 0.6) (layer "F.Cu") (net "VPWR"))
 (via (at 47.6 31) (size 0.8) (drill 0.4) (layers "F.Cu" "B.Cu") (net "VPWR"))
 (via (at 30.1 31) (size 0.8) (drill 0.4) (layers "F.Cu" "B.Cu") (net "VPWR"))
 (via (at 73 31) (size 0.8) (drill 0.4) (layers "F.Cu" "B.Cu") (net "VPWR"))
 (via (at 20 31) (size 0.8) (drill 0.4) (layers "F.Cu" "B.Cu") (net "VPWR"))
 (via (at 35.6 31) (size 0.8) (drill 0.4) (layers "F.Cu" "B.Cu") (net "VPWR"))
 (via (at 46.05 31) (size 0.8) (drill 0.4) (layers "F.Cu" "B.Cu") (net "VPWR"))
 (segment (start 20 31) (end 73 31) (width 1.2) (layer "B.Cu") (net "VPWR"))
 (segment (start 36.5 10) (end 39.4 10) (width 0.35) (layer "F.Cu") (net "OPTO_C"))
 (segment (start 45 10) (end 49.3 10) (width 0.35) (layer "F.Cu") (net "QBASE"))
 (segment (start 49.3 10) (end 49.3 9.05) (width 0.35) (layer "F.Cu") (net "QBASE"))
 (segment (start 45 10) (end 45 14) (width 0.35) (layer "F.Cu") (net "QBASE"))
 (segment (start 45 14) (end 44.4 14) (width 0.35) (layer "F.Cu") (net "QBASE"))
 (segment (start 42.6 10) (end 45 10) (width 0.35) (layer "F.Cu") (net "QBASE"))
 (segment (start 52.7 10) (end 54.4 14) (width 0.35) (layer "F.Cu") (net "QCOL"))
 (segment (start 60.4 18) (end 57.9 18) (width 0.35) (layer "F.Cu") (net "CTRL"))
 (segment (start 57.6 14) (end 60.4 14) (width 0.35) (layer "F.Cu") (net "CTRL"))
 (segment (start 60.4 18) (end 60.4 18) (width 0.35) (layer "F.Cu") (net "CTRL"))
 (segment (start 59 18) (end 59 19.365) (width 0.35) (layer "F.Cu") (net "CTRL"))
 (segment (start 59 19.365) (end 66 19.365) (width 0.35) (layer "F.Cu") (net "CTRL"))
 (segment (start 60.4 18) (end 59 18) (width 0.35) (layer "F.Cu") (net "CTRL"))
 (segment (start 60.4 14) (end 60.4 18) (width 0.35) (layer "F.Cu") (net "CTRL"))
 (segment (start 60.4 18) (end 60.1 23) (width 0.35) (layer "F.Cu") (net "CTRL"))
 (segment (start 66 20.635) (end 68 20.635) (width 1.2) (layer "F.Cu") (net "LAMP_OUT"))
 (via (at 68 20.635) (size 0.8) (drill 0.4) (layers "F.Cu" "B.Cu") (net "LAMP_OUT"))
 (segment (start 12 28) (end 68 28) (width 1.2) (layer "B.Cu") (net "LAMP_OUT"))
 (segment (start 68 20.635) (end 68 28) (width 1.2) (layer "B.Cu") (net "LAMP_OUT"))
 (segment (start 7 27.16) (end 12 27.16) (width 1.2) (layer "B.Cu") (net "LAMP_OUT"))
 (segment (start 12 27.16) (end 12 28) (width 1.2) (layer "B.Cu") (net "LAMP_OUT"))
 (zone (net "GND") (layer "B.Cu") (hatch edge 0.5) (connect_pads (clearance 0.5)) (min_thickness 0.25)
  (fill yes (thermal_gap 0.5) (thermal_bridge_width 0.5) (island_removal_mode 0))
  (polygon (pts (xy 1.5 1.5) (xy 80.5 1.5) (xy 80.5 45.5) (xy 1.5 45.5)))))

